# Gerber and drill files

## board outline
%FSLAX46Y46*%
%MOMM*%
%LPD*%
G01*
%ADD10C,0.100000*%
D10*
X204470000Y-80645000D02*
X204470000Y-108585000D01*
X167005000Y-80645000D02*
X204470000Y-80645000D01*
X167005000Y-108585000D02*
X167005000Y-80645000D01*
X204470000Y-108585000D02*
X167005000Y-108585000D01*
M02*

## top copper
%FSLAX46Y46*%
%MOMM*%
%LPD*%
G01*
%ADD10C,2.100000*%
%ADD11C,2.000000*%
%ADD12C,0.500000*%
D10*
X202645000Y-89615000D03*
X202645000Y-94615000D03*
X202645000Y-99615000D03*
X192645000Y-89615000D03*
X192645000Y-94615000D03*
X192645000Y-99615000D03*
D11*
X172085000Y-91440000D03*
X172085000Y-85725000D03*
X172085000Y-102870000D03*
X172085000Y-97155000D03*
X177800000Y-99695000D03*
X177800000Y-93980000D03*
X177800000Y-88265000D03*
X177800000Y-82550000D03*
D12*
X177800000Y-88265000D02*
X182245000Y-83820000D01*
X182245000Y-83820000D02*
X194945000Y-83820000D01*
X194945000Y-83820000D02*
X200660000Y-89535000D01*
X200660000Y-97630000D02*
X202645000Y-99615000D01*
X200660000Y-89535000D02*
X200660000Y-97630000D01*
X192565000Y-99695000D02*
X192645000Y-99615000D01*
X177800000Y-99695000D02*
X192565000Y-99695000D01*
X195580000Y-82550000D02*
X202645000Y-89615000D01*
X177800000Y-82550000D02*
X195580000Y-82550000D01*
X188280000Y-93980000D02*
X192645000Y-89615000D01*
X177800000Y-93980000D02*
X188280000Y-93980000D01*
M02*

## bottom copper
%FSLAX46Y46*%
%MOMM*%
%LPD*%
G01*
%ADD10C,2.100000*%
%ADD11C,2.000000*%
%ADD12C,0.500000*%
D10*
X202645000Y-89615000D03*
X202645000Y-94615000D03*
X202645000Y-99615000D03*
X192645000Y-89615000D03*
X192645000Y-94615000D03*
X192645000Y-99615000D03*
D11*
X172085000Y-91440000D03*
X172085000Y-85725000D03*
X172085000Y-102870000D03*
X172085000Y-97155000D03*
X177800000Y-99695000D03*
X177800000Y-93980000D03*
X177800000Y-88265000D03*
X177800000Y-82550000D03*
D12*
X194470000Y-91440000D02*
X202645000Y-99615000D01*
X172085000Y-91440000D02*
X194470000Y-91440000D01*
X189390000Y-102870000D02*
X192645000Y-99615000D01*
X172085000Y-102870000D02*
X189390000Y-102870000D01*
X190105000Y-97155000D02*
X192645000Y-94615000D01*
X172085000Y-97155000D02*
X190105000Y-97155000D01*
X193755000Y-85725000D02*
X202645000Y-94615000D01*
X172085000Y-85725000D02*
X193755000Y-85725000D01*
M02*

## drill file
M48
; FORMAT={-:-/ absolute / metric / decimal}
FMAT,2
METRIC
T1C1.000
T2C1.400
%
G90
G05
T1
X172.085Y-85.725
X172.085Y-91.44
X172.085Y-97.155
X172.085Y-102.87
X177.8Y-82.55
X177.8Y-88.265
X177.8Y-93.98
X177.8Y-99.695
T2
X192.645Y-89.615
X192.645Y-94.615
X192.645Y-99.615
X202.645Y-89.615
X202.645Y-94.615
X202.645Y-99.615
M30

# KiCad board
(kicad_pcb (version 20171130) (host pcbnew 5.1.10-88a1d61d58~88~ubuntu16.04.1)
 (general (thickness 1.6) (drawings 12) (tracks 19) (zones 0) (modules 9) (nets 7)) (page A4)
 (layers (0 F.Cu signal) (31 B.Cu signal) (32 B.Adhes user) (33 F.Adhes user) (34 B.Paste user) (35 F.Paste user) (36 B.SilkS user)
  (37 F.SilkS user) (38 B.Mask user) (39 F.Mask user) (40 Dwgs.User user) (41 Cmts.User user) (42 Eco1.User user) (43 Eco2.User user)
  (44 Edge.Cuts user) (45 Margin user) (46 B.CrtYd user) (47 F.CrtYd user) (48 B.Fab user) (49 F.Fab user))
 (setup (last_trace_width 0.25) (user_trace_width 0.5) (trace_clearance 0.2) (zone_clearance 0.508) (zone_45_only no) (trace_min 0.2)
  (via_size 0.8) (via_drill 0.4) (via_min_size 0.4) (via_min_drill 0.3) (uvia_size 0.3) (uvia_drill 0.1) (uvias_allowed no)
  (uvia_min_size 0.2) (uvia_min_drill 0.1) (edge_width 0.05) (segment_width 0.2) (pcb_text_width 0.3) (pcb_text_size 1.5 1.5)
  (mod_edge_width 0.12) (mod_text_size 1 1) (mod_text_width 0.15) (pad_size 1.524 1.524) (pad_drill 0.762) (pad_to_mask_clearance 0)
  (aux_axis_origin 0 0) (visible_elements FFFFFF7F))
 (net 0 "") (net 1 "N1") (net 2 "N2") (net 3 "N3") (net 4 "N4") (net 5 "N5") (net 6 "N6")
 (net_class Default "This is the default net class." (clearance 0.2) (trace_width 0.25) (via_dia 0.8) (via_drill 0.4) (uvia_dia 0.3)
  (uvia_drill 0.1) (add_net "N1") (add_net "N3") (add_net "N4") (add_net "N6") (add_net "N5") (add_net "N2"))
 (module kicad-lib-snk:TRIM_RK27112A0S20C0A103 (layer F.Cu) (at 207.645 94.615)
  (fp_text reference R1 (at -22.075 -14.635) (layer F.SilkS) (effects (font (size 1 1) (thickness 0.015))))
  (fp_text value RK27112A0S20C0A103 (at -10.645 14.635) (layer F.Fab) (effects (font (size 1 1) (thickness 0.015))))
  (pad 3_1 thru_hole circle (at -5 -5) (size 2.1 2.1) (drill 1.4) (layers *.Cu *.Mask) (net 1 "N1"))
  (pad 2_1 thru_hole circle (at -5 0) (size 2.1 2.1) (drill 1.4) (layers *.Cu *.Mask) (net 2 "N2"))
  (pad 1_1 thru_hole circle (at -5 5) (size 2.1 2.1) (drill 1.4) (layers *.Cu *.Mask) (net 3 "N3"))
  (pad 3_2 thru_hole circle (at -15 -5) (size 2.1 2.1) (drill 1.4) (layers *.Cu *.Mask) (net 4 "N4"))
  (pad 2_2 thru_hole circle (at -15 0) (size 2.1 2.1) (drill 1.4) (layers *.Cu *.Mask) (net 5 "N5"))
  (pad 1_2 thru_hole circle (at -15 5) (size 2.1 2.1) (drill 1.4) (layers *.Cu *.Mask) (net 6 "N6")))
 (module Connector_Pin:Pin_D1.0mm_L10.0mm (layer F.Cu) (at 172.085 91.44)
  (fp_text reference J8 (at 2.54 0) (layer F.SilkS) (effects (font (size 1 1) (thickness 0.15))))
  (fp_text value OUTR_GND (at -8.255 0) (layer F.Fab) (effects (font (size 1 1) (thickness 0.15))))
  (pad 1 thru_hole circle (at 0 0) (size 2 2) (drill 1) (layers *.Cu *.Mask) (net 3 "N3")))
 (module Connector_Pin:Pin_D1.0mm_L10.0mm (layer F.Cu) (at 172.085 85.725)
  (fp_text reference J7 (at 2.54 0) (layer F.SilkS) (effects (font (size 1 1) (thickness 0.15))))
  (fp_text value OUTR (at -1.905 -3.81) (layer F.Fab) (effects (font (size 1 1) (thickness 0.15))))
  (pad 1 thru_hole circle (at 0 0) (size 2 2) (drill 1) (layers *.Cu *.Mask) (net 2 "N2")))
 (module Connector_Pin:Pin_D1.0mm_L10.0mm (layer F.Cu) (at 172.085 102.87)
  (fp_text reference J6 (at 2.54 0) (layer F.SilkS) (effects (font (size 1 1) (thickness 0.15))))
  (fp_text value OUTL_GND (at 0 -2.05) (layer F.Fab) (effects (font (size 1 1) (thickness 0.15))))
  (pad 1 thru_hole circle (at 0 0) (size 2 2) (drill 1) (layers *.Cu *.Mask) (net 6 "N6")))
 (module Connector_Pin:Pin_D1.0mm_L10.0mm (layer F.Cu) (at 172.085 97.155)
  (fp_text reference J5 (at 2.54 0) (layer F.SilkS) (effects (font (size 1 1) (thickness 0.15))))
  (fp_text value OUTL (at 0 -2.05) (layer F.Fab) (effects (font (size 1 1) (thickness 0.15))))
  (pad 1 thru_hole circle (at 0 0) (size 2 2) (drill 1) (layers *.Cu *.Mask) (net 5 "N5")))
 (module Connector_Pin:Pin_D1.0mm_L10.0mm (layer F.Cu) (at 177.8 99.695)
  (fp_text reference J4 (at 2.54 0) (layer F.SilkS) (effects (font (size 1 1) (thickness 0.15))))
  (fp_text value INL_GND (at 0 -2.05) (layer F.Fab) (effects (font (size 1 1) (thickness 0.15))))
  (pad 1 thru_hole circle (at 0 0) (size 2 2) (drill 1) (layers *.Cu *.Mask) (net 6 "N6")))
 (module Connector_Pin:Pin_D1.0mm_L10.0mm (layer F.Cu) (at 177.8 93.98)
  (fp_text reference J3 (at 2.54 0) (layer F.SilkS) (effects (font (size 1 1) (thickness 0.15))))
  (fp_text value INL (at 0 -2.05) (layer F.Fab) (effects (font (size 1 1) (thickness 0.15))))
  (pad 1 thru_hole circle (at 0 0) (size 2 2) (drill 1) (layers *.Cu *.Mask) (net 4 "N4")))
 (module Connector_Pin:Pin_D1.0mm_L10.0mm (layer F.Cu) (at 177.8 88.265)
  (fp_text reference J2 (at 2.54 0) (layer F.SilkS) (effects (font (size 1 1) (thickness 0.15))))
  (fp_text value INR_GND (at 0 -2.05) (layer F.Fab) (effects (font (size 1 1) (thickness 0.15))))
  (pad 1 thru_hole circle (at 0 0) (size 2 2) (drill 1) (layers *.Cu *.Mask) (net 3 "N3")))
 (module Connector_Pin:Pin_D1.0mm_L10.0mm (layer F.Cu) (at 177.8 82.55)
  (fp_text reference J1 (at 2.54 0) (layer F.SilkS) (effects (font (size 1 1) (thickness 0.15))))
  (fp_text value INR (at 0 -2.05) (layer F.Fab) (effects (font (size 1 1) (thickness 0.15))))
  (pad 1 thru_hole circle (at 0 0) (size 2 2) (drill 1) (layers *.Cu *.Mask) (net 1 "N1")))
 (gr_line (start 204.47 80.645) (end 204.47 108.585) (layer Edge.Cuts) (width 0.1))
 (gr_line (start 167.005 80.645) (end 204.47 80.645) (layer Edge.Cuts) (width 0.1))
 (gr_line (start 167.005 108.585) (end 167.005 80.645) (layer Edge.Cuts) (width 0.1))
 (gr_line (start 204.47 108.585) (end 167.005 108.585) (layer Edge.Cuts) (width 0.1))
 (segment (start 177.8 88.265) (end 182.245 83.82) (width 0.5) (layer F.Cu) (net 3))
 (segment (start 182.245 83.82) (end 194.945 83.82) (width 0.5) (layer F.Cu) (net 3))
 (segment (start 194.945 83.82) (end 200.66 89.535) (width 0.5) (layer F.Cu) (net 3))
 (segment (start 200.66 97.63) (end 202.645 99.615) (width 0.5) (layer F.Cu) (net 3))
 (segment (start 200.66 89.535) (end 200.66 97.63) (width 0.5) (layer F.Cu) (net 3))
 (segment (start 194.47 91.44) (end 202.645 99.615) (width 0.5) (layer B.Cu) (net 3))
 (segment (start 172.085 91.44) (end 194.47 91.44) (width 0.5) (layer B.Cu) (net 3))
 (segment (start 192.565 99.695) (end 192.645 99.615) (width 0.5) (layer F.Cu) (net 6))
 (segment (start 177.8 99.695) (end 192.565 99.695) (width 0.5) (layer F.Cu) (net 6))
 (segment (start 189.39 102.87) (end 192.645 99.615) (width 0.5) (layer B.Cu) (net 6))
 (segment (start 172.085 102.87) (end 189.39 102.87) (width 0.5) (layer B.Cu) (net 6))
 (segment (start 195.58 82.55) (end 202.645 89.615) (width 0.5) (layer F.Cu) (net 1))
 (segment (start 177.8 82.55) (end 195.58 82.55) (width 0.5) (layer F.Cu) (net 1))
 (segment (start 188.28 93.98) (end 192.645 89.615) (width 0.5) (layer F.Cu) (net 4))
 (segment (start 177.8 93.98) (end 188.28 93.98) (width 0.5) (layer F.Cu) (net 4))
 (segment (start 190.105 97.155) (end 192.645 94.615) (width 0.5) (layer B.Cu) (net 5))
 (segment (start 172.085 97.155) (end 190.105 97.155) (width 0.5) (layer B.Cu) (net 5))
 (segment (start 193.755 85.725) (end 202.645 94.615) (width 0.5) (layer B.Cu) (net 2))
 (segment (start 172.085 85.725) (end 193.755 85.725) (width 0.5) (layer B.Cu) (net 2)))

